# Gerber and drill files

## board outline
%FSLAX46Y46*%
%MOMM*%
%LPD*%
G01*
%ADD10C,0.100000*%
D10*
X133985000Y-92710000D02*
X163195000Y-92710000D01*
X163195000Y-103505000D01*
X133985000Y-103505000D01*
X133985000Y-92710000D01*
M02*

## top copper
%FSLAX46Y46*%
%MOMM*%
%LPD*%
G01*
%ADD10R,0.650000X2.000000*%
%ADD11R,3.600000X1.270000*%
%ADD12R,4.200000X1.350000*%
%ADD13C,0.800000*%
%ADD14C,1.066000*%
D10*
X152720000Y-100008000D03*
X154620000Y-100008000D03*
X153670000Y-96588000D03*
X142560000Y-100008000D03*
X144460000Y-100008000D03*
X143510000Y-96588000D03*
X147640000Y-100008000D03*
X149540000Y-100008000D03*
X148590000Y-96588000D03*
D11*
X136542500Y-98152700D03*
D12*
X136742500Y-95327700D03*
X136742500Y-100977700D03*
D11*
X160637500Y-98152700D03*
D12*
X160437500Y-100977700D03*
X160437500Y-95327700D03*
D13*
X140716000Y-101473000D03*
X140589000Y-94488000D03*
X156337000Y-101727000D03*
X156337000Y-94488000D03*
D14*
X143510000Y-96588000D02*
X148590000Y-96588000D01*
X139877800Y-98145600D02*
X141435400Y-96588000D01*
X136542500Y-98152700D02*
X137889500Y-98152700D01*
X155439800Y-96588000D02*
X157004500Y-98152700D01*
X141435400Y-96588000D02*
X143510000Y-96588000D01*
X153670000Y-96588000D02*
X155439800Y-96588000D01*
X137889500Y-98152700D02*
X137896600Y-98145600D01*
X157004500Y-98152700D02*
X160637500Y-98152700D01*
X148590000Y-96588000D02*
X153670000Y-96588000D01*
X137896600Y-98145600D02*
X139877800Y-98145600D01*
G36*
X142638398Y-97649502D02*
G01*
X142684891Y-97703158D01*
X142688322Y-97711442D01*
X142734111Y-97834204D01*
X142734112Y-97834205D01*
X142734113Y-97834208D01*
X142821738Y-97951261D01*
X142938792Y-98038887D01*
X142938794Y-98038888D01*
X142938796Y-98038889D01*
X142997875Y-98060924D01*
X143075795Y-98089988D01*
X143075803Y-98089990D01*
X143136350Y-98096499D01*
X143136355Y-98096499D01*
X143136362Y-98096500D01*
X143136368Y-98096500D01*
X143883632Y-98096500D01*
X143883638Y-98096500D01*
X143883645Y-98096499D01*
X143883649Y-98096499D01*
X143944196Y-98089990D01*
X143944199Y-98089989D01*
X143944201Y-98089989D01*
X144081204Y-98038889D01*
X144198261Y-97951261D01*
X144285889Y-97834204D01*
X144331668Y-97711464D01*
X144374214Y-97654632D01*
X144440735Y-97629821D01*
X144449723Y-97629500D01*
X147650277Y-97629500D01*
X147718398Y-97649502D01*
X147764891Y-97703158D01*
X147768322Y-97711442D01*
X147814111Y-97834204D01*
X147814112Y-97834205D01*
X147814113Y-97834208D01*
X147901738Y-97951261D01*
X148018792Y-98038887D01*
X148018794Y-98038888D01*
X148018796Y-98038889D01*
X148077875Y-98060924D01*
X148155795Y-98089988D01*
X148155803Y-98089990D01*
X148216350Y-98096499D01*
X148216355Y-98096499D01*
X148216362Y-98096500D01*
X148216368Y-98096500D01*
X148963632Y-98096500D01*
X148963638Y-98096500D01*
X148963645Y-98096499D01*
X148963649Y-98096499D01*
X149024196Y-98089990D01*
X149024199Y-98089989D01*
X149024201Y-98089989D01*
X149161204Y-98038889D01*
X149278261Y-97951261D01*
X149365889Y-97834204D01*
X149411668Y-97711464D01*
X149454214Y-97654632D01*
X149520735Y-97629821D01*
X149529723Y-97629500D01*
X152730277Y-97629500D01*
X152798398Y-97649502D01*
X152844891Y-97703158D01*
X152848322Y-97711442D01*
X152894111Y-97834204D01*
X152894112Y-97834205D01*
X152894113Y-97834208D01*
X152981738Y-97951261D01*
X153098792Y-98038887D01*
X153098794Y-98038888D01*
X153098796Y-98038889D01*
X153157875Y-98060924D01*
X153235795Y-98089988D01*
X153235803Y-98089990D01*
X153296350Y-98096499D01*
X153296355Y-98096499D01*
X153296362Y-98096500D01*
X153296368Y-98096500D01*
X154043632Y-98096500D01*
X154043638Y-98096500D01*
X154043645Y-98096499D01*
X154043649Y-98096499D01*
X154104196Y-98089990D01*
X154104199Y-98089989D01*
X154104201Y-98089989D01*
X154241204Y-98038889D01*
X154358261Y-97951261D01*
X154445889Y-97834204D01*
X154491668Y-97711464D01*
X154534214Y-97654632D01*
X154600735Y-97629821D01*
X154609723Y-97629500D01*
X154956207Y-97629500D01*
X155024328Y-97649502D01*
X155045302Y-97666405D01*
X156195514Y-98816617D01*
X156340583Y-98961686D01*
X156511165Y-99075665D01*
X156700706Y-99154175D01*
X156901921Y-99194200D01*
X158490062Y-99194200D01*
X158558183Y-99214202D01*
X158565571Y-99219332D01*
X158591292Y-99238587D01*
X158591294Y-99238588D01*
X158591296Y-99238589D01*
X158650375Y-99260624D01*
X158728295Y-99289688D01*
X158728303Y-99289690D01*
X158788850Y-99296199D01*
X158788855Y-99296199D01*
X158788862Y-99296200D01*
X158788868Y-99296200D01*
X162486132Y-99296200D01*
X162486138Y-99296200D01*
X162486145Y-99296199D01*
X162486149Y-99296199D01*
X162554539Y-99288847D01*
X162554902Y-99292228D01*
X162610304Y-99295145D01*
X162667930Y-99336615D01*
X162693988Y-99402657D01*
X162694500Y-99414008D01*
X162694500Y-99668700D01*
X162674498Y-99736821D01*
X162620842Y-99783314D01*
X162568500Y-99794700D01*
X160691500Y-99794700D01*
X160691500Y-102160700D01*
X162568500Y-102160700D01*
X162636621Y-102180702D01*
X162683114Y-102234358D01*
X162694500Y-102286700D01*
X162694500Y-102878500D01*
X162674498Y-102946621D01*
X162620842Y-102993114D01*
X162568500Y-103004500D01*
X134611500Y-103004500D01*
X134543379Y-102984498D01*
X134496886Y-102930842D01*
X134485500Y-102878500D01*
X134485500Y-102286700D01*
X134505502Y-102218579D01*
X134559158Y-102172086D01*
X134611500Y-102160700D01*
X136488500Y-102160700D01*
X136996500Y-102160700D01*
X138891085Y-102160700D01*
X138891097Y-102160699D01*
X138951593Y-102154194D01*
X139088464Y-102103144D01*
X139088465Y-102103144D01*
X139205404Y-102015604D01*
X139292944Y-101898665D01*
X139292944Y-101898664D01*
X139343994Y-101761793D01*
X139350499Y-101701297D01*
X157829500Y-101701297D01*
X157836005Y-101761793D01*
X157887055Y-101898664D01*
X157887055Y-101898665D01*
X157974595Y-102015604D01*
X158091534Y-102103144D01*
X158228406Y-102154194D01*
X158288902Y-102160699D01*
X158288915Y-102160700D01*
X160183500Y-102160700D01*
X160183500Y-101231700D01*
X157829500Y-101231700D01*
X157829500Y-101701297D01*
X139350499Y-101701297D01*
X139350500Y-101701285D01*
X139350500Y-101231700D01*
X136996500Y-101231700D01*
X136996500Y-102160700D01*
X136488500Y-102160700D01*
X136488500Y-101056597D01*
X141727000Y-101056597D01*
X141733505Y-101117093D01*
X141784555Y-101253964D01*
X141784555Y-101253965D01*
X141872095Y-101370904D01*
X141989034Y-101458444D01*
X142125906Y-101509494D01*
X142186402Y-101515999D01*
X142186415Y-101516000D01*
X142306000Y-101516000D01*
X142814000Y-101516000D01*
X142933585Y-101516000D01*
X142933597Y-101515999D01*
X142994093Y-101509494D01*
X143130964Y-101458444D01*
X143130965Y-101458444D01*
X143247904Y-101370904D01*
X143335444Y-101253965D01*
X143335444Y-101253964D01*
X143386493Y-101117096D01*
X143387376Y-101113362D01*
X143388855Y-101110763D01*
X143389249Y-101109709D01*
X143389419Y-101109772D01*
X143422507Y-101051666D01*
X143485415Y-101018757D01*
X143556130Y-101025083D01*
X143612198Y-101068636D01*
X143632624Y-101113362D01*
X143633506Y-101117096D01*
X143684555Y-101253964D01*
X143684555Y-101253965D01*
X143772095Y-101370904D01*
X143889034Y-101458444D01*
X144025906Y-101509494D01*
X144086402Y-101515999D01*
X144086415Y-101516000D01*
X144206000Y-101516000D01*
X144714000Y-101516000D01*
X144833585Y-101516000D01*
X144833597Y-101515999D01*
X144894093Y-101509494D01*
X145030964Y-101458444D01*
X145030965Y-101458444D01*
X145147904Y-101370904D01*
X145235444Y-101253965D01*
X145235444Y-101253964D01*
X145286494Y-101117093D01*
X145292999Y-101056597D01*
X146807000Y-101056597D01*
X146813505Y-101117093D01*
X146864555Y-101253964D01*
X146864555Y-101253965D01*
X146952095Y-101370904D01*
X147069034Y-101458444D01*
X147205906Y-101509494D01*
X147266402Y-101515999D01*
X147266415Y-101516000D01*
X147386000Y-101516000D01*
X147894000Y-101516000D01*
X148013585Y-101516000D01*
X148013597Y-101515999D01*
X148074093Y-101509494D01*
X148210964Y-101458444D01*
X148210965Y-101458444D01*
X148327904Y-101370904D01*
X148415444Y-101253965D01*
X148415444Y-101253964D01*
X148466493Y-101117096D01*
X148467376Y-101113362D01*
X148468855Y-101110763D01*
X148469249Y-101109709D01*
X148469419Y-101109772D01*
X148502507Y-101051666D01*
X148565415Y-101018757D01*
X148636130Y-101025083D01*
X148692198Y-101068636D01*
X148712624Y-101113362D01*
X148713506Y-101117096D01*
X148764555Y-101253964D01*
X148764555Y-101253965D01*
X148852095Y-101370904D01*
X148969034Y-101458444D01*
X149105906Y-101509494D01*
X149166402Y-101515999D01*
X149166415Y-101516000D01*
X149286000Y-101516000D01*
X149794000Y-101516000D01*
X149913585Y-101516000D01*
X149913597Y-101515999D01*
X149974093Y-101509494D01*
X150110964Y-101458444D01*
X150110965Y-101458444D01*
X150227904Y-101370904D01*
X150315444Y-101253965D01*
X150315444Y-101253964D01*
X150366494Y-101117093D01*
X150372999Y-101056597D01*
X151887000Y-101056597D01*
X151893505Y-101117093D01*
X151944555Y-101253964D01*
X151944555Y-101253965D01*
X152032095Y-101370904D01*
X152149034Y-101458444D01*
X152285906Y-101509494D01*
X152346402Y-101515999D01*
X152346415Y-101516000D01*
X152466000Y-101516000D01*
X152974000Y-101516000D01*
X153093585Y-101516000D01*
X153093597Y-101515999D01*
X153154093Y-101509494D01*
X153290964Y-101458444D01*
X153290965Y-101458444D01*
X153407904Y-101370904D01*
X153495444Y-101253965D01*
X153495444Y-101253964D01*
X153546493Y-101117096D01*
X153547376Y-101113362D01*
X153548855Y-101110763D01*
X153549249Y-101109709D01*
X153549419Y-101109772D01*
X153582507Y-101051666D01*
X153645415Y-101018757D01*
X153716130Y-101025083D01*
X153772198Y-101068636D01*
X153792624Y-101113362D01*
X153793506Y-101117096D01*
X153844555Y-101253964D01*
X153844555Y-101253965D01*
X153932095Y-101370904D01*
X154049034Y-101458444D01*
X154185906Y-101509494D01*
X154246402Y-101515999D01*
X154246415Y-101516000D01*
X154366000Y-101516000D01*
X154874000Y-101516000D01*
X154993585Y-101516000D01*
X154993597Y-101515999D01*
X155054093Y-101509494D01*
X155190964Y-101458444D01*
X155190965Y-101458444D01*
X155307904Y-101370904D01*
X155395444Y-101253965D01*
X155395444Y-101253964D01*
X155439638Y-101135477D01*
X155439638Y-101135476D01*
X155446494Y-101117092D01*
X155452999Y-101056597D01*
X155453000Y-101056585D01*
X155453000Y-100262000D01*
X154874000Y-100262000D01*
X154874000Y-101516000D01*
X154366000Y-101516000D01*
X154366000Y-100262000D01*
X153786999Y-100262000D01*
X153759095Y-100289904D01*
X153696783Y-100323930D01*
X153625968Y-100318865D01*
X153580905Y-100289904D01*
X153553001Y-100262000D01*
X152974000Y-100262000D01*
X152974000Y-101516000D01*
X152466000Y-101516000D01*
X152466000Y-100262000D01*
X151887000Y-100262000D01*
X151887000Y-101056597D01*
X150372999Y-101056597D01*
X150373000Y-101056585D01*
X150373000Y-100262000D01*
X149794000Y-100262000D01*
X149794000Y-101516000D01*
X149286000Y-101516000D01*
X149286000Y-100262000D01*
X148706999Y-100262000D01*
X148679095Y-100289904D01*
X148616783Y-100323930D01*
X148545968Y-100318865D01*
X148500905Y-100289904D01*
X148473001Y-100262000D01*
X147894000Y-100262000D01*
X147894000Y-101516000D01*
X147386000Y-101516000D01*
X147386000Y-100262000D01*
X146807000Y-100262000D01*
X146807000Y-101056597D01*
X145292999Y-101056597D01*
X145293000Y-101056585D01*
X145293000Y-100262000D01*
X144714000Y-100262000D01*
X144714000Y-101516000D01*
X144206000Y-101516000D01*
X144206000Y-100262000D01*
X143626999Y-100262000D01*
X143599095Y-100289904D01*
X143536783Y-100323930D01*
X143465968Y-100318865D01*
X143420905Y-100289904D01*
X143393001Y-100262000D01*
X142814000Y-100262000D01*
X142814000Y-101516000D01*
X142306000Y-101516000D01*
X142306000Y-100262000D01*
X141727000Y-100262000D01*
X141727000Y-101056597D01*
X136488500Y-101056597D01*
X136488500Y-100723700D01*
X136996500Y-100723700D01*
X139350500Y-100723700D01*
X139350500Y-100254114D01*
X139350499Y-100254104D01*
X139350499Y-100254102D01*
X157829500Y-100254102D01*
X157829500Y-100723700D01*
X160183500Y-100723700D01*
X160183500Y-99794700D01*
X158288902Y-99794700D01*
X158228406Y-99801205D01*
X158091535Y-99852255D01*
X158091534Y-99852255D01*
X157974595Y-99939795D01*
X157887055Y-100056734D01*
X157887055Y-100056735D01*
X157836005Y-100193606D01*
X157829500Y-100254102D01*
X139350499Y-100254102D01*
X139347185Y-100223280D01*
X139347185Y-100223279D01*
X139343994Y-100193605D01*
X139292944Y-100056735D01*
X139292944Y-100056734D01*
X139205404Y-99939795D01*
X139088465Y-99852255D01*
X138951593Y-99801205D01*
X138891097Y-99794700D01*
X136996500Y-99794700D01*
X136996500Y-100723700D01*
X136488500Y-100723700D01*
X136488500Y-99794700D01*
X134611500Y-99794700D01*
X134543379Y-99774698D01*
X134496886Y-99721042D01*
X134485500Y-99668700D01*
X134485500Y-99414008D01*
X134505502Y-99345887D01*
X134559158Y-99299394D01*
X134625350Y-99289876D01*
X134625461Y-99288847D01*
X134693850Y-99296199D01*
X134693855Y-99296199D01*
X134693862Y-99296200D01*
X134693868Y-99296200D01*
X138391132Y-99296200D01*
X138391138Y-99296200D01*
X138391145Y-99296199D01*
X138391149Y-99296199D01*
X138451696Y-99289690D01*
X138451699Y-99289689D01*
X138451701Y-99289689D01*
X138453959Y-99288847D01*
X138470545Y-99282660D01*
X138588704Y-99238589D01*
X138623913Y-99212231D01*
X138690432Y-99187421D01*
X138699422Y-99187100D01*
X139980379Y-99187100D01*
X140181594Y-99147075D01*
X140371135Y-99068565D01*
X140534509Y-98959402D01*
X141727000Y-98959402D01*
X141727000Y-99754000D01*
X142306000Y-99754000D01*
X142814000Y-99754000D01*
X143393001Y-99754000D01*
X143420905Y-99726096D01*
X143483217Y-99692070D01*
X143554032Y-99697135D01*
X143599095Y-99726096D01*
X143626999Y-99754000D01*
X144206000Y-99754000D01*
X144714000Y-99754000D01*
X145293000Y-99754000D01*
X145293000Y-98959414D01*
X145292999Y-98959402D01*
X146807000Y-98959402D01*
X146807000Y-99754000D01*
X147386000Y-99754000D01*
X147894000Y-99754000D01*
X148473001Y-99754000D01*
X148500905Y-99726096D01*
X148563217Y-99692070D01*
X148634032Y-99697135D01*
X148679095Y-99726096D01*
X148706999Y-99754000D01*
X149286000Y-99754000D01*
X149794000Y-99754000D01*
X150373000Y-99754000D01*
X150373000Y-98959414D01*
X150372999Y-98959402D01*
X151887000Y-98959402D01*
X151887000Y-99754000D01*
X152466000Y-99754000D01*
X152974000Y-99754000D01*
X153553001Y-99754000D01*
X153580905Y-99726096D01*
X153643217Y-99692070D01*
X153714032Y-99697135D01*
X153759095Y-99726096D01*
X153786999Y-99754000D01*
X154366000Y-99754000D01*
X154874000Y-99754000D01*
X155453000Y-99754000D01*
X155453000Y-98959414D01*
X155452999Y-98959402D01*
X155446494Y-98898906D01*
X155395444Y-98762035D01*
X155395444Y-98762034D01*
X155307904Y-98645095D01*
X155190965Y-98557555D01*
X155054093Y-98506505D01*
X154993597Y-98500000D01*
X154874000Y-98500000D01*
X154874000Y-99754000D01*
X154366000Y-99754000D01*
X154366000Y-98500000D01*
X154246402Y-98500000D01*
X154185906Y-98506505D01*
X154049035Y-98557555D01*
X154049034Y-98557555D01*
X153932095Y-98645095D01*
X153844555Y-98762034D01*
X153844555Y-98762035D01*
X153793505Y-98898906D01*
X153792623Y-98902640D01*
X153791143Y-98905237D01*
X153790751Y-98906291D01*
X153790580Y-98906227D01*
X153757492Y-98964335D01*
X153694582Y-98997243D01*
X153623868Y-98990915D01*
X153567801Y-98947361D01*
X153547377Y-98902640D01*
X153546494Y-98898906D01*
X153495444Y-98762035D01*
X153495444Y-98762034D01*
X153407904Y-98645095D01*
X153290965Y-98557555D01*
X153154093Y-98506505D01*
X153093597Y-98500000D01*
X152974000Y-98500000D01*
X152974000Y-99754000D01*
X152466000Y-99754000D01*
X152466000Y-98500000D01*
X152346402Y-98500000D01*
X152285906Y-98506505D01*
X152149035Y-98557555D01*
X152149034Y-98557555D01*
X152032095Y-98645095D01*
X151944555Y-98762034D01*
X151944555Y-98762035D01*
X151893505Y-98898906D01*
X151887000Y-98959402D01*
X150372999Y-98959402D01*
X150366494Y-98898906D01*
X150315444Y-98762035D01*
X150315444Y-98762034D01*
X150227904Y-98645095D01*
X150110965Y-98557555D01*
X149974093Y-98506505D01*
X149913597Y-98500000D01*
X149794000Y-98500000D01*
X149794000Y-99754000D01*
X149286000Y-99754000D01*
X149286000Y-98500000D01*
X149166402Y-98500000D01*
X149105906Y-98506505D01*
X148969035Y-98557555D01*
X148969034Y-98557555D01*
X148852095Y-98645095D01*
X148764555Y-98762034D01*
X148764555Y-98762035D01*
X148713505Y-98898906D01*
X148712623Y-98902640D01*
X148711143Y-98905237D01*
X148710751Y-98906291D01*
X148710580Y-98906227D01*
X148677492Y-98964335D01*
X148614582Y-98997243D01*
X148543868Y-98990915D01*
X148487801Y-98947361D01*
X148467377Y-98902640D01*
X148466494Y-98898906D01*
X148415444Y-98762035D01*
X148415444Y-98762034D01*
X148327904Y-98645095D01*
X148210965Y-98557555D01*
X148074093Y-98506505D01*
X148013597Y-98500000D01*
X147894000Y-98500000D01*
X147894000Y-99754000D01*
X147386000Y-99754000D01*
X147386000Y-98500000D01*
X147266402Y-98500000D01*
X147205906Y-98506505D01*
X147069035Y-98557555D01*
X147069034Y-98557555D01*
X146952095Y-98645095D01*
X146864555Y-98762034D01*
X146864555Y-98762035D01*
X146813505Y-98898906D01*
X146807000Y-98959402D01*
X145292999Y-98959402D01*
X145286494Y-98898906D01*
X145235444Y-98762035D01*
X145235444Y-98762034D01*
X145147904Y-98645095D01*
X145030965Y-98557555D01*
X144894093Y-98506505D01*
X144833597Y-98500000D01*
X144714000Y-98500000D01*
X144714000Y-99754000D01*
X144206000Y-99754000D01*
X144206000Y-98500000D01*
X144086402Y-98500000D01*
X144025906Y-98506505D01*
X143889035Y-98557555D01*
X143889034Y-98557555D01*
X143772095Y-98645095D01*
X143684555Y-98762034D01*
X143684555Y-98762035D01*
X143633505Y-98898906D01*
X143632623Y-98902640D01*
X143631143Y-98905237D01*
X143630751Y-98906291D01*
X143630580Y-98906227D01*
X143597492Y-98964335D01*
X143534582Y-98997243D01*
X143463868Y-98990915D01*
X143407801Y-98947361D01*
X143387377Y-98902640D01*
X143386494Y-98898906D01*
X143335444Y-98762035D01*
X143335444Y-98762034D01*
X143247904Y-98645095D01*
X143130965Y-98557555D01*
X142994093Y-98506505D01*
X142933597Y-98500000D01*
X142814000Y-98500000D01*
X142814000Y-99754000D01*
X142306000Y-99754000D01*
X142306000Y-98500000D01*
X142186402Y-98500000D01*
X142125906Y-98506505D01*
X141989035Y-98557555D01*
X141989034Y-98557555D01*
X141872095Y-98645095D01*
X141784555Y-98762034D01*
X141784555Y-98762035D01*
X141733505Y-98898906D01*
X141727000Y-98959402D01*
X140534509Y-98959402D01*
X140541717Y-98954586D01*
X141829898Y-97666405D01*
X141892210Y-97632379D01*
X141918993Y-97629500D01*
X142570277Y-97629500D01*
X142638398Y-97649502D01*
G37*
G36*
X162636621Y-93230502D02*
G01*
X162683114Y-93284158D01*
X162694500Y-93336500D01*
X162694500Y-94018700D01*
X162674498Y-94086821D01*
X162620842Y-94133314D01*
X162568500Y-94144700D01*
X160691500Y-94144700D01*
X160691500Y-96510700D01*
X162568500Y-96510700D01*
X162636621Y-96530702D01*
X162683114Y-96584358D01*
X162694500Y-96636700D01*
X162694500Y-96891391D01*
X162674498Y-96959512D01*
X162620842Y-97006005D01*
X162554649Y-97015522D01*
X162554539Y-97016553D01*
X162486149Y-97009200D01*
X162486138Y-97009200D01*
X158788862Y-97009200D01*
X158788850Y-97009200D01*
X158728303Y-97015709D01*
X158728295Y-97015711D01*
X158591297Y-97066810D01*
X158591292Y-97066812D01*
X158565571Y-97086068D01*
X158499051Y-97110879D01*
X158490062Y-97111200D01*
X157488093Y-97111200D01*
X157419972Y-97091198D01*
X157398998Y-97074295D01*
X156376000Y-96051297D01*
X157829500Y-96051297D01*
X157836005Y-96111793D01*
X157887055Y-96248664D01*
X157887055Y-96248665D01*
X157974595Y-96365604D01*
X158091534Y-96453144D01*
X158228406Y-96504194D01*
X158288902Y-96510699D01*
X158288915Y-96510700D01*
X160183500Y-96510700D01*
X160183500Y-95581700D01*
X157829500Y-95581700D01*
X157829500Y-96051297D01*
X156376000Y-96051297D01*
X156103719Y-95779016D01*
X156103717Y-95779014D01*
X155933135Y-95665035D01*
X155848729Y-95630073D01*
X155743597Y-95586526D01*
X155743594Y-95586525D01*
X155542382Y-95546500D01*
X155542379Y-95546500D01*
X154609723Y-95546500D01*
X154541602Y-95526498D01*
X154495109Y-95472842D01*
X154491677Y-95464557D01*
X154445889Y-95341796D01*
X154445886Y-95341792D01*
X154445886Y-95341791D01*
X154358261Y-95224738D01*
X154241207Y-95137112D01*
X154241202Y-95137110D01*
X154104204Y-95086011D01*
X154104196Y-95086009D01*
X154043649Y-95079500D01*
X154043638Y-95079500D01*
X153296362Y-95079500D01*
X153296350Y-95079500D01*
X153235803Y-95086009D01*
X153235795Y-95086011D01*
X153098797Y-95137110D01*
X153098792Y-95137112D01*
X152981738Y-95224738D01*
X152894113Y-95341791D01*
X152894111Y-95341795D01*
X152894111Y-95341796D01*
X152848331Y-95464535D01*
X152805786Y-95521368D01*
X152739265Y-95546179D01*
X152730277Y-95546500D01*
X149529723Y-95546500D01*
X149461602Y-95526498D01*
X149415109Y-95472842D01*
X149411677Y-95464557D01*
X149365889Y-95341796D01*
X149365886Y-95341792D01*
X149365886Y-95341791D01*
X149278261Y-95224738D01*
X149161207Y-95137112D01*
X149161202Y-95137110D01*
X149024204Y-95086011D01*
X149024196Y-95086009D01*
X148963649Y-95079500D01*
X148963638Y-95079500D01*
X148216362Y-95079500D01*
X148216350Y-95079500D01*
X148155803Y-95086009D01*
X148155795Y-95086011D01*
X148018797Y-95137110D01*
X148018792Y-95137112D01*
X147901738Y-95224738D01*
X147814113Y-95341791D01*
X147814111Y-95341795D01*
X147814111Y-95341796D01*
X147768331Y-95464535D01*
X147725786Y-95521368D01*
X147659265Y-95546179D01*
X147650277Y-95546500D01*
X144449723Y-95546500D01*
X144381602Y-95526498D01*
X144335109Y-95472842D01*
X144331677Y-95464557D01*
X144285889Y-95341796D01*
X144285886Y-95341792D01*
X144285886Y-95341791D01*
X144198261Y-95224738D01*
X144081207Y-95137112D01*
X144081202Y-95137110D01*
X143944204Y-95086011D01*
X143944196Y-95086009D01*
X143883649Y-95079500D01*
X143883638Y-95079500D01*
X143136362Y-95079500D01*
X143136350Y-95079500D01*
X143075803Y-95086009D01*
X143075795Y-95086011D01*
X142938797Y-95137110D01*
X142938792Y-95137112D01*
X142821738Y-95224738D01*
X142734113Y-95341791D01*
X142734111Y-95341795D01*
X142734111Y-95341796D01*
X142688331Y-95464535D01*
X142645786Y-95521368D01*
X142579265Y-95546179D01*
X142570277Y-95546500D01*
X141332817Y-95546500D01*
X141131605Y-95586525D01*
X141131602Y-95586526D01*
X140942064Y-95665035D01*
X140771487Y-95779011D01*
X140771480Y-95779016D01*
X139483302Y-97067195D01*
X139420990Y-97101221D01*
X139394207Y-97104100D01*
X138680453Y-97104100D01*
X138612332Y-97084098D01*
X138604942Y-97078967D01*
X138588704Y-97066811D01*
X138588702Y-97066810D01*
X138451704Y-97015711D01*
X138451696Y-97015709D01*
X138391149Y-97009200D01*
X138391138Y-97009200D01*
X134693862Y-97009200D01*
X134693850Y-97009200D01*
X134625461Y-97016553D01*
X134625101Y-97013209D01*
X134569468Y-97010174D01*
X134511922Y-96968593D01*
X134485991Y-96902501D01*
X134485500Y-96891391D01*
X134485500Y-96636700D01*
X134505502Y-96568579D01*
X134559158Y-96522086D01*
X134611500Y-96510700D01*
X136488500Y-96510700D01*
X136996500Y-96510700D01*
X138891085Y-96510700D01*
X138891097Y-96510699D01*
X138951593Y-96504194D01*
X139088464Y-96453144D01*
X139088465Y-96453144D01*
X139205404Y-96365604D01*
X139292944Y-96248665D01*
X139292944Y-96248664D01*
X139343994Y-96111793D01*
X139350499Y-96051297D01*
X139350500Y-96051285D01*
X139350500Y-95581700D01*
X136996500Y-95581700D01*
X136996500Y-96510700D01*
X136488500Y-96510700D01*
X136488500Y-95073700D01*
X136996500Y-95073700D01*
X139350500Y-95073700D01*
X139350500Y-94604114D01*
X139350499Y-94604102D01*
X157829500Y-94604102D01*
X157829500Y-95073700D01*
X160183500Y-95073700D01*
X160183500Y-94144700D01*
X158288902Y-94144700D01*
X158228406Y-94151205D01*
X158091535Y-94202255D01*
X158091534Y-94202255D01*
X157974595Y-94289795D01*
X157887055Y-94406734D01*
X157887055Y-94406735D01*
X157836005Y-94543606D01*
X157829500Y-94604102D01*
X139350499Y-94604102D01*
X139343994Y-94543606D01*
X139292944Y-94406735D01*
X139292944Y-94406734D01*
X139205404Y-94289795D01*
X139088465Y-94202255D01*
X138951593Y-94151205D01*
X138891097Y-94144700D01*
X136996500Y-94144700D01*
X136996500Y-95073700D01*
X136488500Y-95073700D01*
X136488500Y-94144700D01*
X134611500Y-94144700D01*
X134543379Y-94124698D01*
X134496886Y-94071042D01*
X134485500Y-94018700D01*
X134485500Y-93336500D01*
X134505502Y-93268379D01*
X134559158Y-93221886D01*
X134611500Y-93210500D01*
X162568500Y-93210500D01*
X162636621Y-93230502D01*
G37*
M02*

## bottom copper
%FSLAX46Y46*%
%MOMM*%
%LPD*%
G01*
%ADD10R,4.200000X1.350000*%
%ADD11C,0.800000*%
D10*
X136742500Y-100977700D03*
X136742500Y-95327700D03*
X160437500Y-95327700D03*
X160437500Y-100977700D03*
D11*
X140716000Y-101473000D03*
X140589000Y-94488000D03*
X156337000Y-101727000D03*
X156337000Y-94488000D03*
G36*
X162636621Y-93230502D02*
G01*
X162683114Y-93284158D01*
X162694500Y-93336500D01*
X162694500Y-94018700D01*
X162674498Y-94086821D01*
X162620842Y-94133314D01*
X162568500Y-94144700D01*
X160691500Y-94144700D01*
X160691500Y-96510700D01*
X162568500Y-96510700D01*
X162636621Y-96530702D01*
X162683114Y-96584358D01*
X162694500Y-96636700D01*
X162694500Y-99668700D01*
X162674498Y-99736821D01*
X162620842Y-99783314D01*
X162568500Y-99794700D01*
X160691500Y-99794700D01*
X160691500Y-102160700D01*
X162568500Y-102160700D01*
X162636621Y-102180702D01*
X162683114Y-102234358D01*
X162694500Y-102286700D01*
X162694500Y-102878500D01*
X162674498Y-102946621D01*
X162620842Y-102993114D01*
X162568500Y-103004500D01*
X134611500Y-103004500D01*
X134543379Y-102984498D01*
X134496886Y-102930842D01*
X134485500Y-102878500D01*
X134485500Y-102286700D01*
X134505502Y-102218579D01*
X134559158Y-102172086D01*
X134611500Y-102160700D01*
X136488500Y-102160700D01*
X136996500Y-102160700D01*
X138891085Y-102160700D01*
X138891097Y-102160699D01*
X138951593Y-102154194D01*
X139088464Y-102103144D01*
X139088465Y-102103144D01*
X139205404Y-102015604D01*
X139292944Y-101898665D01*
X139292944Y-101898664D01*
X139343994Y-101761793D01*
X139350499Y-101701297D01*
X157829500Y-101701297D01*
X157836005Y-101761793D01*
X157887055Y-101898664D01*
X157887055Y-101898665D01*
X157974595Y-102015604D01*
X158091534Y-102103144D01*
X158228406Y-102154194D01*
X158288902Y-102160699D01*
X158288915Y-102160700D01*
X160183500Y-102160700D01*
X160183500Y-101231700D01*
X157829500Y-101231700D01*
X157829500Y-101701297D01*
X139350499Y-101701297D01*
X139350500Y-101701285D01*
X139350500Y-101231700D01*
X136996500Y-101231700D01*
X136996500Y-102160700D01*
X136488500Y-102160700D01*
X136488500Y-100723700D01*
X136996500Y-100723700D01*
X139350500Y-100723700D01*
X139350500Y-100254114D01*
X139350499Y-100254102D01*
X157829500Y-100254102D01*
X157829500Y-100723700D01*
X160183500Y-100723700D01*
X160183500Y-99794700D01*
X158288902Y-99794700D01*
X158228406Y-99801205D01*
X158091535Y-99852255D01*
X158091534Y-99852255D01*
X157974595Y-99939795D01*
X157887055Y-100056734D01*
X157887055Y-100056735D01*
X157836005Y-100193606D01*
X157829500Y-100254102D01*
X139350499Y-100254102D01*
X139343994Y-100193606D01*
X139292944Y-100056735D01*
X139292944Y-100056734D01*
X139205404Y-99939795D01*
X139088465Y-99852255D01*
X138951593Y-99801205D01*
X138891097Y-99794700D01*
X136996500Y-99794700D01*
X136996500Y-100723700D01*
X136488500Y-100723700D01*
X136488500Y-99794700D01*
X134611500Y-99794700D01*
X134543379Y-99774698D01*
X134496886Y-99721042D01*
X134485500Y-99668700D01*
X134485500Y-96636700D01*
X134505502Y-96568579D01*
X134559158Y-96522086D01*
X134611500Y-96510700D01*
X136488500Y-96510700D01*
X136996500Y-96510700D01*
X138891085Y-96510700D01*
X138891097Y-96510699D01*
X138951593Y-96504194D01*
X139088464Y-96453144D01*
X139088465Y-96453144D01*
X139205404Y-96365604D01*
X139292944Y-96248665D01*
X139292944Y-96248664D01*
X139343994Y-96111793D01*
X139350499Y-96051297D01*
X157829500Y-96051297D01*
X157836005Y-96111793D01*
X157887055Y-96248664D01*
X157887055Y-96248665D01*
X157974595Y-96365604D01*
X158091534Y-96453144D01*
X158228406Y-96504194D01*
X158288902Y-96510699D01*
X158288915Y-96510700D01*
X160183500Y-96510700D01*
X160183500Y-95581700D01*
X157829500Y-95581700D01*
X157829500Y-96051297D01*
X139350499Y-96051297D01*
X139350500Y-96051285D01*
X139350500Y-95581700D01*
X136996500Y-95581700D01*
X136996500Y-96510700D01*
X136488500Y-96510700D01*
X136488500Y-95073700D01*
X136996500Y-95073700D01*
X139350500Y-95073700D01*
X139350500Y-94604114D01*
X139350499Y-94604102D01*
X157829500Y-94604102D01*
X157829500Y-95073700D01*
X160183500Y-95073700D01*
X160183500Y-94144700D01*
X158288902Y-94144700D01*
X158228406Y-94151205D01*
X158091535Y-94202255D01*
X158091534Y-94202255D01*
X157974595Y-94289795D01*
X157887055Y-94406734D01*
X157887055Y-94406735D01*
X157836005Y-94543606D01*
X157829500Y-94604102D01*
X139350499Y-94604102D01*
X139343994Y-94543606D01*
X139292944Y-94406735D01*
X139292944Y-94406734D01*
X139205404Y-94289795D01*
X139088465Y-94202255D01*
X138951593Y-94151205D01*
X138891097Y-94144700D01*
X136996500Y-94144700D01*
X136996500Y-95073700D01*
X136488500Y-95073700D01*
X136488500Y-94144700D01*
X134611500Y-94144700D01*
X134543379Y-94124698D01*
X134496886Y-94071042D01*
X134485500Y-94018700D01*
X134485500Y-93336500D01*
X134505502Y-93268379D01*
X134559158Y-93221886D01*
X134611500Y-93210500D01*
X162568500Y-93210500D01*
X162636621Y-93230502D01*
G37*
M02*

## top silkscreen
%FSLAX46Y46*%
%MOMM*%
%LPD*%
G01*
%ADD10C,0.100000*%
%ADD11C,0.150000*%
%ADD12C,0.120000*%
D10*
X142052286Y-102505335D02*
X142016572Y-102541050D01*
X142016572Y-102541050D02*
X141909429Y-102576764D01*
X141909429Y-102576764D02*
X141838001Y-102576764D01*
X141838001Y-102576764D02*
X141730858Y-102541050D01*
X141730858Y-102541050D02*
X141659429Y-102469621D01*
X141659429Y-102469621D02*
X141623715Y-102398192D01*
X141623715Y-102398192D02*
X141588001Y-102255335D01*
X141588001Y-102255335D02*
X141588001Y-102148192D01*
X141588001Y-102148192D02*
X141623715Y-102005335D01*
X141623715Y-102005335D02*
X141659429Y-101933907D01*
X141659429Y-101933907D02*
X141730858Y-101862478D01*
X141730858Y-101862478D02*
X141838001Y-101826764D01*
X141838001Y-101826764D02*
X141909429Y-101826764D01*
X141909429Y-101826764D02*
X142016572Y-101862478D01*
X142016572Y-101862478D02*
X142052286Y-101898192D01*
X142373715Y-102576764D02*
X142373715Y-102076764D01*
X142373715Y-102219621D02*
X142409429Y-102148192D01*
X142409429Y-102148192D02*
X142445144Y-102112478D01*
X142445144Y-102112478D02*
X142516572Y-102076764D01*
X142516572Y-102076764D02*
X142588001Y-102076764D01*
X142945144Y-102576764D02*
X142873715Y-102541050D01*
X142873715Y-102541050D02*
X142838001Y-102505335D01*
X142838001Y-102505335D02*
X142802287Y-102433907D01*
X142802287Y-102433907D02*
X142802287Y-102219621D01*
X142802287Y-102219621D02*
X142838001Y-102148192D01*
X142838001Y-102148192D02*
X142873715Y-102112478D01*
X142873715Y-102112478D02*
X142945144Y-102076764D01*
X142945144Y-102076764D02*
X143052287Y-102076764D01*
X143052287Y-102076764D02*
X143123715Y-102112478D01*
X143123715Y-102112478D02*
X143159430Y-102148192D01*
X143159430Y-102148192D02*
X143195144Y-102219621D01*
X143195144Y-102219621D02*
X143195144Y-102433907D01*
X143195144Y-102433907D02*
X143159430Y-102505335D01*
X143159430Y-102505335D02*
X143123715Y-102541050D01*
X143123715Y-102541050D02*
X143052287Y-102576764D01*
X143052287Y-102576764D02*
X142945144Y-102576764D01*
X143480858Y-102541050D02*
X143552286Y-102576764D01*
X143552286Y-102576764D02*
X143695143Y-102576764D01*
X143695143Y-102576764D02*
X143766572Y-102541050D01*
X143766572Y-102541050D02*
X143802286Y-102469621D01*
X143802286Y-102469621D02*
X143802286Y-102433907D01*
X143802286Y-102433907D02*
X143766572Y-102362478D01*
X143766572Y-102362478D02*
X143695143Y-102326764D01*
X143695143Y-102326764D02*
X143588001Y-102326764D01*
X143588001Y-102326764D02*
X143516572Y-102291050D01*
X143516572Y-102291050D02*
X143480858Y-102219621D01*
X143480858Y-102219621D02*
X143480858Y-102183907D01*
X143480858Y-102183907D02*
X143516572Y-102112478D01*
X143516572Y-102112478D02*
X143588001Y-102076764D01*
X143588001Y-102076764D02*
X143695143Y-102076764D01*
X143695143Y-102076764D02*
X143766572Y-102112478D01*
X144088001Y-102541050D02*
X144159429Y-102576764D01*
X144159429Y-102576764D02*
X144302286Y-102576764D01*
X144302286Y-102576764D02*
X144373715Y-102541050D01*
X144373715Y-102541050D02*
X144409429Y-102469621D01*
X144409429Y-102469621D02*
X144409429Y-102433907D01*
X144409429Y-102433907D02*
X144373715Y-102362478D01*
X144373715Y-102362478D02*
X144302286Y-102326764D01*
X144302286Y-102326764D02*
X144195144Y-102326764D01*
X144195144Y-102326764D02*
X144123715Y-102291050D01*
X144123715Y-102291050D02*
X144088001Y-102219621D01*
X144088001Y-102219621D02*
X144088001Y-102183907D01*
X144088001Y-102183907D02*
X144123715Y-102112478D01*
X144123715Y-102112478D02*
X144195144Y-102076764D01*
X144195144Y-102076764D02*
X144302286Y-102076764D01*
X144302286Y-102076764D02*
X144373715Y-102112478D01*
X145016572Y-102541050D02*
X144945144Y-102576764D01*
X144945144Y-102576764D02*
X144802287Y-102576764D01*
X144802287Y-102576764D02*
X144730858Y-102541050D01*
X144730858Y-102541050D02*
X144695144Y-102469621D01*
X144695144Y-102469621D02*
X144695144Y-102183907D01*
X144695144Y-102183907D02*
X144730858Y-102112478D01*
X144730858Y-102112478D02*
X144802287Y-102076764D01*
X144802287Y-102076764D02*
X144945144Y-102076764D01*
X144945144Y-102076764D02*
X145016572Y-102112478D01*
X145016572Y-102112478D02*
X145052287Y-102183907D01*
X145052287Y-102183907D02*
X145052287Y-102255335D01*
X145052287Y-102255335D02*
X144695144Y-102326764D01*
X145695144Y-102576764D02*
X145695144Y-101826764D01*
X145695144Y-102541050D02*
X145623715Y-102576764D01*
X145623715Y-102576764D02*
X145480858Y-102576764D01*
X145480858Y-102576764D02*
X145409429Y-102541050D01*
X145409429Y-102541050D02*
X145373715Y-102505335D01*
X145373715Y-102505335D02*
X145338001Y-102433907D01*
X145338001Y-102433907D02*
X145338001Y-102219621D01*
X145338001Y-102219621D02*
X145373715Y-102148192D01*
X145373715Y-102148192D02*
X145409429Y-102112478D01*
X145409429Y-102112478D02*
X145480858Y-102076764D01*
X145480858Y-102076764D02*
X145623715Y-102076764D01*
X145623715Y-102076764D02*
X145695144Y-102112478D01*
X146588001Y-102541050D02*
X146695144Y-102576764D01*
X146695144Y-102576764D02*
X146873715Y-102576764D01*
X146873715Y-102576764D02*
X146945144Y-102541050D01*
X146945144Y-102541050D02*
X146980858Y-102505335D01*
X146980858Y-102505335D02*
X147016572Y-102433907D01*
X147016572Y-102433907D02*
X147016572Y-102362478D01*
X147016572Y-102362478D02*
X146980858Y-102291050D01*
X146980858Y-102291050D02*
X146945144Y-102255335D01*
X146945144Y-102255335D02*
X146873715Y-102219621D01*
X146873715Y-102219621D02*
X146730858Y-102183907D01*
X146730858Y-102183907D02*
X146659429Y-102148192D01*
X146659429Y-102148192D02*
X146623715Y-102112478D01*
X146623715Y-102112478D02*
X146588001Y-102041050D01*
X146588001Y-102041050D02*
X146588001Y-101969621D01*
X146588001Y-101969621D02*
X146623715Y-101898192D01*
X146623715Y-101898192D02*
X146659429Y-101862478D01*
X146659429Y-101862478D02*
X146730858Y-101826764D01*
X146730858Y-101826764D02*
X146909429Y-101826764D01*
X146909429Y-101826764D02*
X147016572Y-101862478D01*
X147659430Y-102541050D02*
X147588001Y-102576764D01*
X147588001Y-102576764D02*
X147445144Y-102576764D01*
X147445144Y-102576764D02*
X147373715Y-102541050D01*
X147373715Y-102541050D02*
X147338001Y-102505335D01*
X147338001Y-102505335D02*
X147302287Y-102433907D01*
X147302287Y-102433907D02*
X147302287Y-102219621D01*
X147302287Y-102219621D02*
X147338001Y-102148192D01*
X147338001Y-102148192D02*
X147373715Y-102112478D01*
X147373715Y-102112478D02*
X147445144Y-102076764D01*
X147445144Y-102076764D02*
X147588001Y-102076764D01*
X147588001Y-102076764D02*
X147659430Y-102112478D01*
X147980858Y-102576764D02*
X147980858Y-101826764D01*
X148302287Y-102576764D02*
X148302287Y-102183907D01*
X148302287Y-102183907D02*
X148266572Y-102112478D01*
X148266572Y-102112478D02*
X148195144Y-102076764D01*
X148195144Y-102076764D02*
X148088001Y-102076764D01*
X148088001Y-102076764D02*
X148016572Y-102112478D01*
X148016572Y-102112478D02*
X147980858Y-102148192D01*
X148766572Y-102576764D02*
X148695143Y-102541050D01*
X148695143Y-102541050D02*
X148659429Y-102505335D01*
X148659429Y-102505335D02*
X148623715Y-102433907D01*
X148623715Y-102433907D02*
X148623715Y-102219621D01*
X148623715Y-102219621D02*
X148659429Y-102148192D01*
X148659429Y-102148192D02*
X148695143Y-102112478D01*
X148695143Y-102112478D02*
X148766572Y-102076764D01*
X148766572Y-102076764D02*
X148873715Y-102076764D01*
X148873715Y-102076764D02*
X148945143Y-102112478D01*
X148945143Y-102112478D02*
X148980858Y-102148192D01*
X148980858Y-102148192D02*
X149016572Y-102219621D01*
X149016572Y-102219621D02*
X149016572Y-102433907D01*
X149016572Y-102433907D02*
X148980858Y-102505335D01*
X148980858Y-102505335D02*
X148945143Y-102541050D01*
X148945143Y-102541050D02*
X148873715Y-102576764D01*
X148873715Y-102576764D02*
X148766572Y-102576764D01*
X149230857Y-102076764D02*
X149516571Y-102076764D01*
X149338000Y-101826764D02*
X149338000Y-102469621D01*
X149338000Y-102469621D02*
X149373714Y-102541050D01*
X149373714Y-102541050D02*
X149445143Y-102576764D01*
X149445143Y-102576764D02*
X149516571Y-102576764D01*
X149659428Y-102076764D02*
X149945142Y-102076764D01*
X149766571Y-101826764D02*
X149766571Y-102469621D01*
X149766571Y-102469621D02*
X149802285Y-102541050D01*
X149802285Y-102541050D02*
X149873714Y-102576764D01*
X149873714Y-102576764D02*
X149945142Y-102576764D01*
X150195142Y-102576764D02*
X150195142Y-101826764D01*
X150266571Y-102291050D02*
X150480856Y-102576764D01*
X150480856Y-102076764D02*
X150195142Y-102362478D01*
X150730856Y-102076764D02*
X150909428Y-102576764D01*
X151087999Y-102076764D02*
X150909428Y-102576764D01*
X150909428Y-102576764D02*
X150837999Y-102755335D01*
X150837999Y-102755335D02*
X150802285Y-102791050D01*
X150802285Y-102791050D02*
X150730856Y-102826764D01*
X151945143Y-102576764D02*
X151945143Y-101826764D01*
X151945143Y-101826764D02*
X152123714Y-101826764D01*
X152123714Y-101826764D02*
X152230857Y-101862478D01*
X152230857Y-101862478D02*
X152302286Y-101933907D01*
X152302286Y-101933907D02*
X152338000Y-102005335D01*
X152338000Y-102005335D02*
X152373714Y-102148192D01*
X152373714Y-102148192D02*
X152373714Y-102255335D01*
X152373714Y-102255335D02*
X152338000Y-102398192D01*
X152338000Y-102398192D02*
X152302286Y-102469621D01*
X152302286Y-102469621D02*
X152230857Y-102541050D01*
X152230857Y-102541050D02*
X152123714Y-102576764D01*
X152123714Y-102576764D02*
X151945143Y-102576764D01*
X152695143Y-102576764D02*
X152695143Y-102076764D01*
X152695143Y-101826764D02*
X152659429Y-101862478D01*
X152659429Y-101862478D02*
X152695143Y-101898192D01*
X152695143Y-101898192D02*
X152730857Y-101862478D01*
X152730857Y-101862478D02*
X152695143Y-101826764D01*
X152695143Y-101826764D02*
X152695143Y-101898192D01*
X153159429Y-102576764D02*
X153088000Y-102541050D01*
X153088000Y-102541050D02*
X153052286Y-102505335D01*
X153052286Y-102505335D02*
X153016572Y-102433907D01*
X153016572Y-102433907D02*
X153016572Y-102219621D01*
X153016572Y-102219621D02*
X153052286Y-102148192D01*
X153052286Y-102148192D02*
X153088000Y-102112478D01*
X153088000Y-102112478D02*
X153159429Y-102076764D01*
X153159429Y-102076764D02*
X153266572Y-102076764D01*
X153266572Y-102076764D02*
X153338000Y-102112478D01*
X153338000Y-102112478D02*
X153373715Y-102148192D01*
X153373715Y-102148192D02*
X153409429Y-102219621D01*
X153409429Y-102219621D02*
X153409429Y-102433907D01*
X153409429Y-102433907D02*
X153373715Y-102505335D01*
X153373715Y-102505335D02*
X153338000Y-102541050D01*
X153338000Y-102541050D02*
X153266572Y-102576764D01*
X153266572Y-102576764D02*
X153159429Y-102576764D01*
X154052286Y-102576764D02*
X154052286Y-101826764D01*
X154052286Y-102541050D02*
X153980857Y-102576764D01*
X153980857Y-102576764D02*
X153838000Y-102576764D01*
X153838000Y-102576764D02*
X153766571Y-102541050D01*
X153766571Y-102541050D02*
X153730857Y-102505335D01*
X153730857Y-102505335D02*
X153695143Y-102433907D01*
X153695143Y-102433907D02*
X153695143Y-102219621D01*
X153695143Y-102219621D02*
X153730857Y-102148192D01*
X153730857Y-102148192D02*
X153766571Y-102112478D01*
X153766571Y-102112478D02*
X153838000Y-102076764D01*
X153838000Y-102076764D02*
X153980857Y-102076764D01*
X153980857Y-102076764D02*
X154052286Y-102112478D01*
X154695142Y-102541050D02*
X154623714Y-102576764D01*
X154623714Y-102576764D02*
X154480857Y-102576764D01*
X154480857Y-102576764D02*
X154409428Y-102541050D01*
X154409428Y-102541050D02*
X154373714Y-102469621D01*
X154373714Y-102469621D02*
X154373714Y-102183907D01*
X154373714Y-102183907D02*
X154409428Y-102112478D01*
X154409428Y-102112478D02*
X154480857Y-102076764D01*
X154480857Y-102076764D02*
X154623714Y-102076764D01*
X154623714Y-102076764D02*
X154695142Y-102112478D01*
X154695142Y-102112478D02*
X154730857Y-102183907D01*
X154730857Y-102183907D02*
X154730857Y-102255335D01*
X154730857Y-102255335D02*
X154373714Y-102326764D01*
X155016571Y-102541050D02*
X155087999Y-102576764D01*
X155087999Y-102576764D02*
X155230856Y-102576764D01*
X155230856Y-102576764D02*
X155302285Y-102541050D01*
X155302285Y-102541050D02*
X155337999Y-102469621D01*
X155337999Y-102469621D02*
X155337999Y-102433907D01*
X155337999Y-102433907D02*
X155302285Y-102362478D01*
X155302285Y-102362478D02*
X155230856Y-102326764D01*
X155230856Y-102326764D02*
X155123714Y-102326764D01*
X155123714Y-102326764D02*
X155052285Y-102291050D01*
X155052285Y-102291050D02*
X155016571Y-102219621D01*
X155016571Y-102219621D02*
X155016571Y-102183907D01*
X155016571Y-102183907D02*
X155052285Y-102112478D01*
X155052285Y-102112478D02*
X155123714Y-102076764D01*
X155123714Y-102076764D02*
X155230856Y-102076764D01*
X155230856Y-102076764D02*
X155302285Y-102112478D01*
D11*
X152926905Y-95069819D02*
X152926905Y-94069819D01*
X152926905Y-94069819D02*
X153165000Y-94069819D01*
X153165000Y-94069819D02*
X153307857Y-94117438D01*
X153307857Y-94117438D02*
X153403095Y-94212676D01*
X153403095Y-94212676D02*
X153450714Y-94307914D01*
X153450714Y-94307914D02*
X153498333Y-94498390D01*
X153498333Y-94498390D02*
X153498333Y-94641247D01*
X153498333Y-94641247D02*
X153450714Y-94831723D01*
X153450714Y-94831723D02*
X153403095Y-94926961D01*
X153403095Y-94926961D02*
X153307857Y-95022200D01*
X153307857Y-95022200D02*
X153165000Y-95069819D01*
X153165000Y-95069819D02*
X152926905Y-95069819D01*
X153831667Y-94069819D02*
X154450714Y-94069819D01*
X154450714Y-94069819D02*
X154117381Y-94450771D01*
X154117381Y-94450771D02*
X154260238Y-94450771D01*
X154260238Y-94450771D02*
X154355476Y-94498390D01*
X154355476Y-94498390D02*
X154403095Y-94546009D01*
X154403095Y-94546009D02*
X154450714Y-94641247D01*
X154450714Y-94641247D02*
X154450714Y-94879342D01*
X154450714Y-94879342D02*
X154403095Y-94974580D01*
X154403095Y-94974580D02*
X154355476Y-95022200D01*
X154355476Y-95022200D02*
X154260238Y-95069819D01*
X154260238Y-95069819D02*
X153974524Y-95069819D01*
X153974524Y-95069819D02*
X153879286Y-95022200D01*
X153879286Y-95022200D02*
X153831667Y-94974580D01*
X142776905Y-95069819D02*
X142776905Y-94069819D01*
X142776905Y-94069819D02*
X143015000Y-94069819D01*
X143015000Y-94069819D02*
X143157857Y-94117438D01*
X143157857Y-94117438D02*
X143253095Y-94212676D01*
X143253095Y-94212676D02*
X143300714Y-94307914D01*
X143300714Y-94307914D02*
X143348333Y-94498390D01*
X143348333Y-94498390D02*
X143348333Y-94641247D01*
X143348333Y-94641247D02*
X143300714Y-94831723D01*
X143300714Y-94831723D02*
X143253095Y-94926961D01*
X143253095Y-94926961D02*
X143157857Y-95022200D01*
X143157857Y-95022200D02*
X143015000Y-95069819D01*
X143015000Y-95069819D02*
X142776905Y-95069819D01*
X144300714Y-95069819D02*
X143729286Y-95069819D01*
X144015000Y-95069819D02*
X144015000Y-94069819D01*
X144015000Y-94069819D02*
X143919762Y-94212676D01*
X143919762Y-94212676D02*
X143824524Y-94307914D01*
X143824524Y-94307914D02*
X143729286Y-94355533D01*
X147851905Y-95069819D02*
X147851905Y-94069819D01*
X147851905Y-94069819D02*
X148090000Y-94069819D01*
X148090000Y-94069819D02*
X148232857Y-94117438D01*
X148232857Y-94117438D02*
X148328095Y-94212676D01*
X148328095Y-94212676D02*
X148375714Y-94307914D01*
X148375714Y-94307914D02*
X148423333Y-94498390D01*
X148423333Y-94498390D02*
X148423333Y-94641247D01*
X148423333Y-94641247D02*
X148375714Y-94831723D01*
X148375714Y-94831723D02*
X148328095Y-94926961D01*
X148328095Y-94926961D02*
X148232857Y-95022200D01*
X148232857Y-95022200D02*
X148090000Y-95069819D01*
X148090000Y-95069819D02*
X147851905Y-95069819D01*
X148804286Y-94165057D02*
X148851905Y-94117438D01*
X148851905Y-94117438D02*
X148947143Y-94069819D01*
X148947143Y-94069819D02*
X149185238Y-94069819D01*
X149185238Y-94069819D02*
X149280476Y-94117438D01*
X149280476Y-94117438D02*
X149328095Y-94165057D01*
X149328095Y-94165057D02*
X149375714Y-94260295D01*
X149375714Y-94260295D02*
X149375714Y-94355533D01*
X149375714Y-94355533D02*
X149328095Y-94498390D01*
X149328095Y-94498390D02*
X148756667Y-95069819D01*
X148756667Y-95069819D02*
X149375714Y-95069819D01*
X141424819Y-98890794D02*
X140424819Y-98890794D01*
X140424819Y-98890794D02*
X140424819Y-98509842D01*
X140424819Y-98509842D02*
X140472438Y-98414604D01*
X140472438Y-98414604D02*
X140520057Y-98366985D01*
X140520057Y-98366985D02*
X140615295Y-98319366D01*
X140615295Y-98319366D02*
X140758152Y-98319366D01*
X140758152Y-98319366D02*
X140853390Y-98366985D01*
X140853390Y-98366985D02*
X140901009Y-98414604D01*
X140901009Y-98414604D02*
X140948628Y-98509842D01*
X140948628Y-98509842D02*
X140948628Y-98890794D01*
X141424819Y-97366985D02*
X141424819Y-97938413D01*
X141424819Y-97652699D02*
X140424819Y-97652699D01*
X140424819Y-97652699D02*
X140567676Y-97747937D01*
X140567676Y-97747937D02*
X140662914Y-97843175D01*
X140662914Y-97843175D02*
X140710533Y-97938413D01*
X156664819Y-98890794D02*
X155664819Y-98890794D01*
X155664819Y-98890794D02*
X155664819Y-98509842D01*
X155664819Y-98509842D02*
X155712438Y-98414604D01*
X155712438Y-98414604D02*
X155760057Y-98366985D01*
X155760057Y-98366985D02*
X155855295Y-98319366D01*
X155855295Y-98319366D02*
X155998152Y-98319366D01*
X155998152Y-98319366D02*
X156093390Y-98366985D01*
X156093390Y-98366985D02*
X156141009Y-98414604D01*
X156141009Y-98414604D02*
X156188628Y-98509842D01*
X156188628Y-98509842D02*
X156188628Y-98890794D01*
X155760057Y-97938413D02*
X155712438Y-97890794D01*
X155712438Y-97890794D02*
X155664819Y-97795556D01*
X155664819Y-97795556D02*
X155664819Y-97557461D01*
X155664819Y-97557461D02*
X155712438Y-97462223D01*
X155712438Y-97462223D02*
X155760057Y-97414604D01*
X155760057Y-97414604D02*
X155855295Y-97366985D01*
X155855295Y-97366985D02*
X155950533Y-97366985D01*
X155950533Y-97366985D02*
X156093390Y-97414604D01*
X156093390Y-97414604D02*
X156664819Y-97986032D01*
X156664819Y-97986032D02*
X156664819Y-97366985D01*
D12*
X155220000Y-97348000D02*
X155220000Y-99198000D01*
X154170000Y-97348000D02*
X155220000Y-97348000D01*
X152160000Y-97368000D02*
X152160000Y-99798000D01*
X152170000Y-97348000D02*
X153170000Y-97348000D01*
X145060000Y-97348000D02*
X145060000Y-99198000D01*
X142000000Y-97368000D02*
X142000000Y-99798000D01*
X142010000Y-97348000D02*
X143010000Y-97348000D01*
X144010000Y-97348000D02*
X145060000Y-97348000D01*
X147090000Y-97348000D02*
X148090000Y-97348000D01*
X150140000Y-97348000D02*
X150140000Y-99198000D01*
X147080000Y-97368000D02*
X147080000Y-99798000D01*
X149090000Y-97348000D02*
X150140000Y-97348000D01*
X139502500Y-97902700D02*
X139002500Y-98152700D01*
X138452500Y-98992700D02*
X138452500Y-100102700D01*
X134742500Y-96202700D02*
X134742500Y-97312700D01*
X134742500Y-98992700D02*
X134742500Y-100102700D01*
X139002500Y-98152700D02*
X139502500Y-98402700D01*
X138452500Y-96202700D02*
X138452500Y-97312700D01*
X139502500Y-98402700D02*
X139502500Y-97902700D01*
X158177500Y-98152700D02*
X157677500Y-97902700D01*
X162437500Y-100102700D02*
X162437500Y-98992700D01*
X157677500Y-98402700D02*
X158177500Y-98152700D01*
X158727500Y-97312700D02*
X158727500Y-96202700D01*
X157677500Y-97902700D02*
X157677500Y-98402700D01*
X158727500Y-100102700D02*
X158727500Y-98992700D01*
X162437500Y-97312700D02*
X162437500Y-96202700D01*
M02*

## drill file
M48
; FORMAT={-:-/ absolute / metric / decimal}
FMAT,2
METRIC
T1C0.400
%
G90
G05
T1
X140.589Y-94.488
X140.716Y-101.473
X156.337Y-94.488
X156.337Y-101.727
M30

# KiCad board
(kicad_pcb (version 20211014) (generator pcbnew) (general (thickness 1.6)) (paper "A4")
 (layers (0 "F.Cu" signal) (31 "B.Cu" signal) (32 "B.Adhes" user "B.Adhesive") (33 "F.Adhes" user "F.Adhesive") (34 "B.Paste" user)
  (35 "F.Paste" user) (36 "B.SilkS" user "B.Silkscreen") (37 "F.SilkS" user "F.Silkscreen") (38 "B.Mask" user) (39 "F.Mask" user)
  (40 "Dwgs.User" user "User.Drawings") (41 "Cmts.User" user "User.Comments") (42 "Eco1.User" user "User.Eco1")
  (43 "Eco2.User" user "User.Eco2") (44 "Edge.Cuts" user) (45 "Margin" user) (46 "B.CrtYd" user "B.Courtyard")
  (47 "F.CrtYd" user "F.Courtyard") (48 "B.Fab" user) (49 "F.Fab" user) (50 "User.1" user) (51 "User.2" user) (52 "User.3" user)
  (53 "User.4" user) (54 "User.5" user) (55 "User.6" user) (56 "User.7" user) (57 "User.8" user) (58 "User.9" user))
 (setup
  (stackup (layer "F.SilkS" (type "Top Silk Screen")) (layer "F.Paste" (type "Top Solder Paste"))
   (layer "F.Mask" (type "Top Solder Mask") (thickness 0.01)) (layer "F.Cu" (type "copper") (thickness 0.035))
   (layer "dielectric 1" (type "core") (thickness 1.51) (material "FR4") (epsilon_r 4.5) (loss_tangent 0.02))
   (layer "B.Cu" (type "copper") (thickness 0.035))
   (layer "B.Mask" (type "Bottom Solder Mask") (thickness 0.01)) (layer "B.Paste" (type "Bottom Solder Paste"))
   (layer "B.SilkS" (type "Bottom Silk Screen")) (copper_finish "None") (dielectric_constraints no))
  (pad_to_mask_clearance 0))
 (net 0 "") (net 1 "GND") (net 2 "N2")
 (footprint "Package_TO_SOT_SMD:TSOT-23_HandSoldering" (layer "F.Cu") (at 153.67 98.298 90)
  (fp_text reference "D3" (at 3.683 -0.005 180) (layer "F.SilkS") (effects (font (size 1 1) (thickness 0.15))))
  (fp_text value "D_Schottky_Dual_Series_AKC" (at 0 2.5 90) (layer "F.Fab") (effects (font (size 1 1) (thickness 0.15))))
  (fp_line (start 0.95 1.55) (end -0.9 1.55) (layer "F.SilkS") (width 0.12))
  (fp_line (start 0.95 0.5) (end 0.95 1.55) (layer "F.SilkS") (width 0.12))
  (fp_line (start 0.93 -1.51) (end -1.5 -1.51) (layer "F.SilkS") (width 0.12))
  (fp_line (start 0.95 -1.5) (end 0.95 -0.5) (layer "F.SilkS") (width 0.12))
  (pad "1" smd rect (at -1.71 -0.95 90) (size 2 0.65) (layers "F.Cu" "F.Paste" "F.Mask") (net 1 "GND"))
  (pad "2" smd rect (at -1.71 0.95 90) (size 2 0.65) (layers "F.Cu" "F.Paste" "F.Mask") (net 1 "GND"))
  (pad "D3" smd rect (at 1.71 0 90) (size 2 0.65) (layers "F.Cu" "F.Paste" "F.Mask") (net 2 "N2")))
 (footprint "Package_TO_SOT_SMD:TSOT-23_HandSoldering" (layer "F.Cu") (at 143.51 98.298 90)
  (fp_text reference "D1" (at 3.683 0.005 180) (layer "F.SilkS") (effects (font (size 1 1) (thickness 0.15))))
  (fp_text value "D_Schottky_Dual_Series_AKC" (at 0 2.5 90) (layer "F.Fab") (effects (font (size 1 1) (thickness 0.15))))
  (fp_line (start 0.95 1.55) (end -0.9 1.55) (layer "F.SilkS") (width 0.12))
  (fp_line (start 0.93 -1.51) (end -1.5 -1.51) (layer "F.SilkS") (width 0.12))
  (fp_line (start 0.95 -1.5) (end 0.95 -0.5) (layer "F.SilkS") (width 0.12))
  (fp_line (start 0.95 0.5) (end 0.95 1.55) (layer "F.SilkS") (width 0.12))
  (pad "1" smd rect (at -1.71 -0.95 90) (size 2 0.65) (layers "F.Cu" "F.Paste" "F.Mask") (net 1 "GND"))
  (pad "2" smd rect (at -1.71 0.95 90) (size 2 0.65) (layers "F.Cu" "F.Paste" "F.Mask") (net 1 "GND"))
  (pad "3" smd rect (at 1.71 0 90) (size 2 0.65) (layers "F.Cu" "F.Paste" "F.Mask") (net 2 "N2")))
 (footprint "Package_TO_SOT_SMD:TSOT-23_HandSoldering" (layer "F.Cu") (at 148.59 98.298 90)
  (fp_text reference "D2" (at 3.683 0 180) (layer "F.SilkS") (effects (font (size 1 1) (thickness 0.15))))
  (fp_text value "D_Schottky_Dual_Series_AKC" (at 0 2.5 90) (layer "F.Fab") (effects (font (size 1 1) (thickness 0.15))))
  (fp_line (start 0.95 -1.5) (end 0.95 -0.5) (layer "F.SilkS") (width 0.12))
  (fp_line (start 0.95 1.55) (end -0.9 1.55) (layer "F.SilkS") (width 0.12))
  (fp_line (start 0.93 -1.51) (end -1.5 -1.51) (layer "F.SilkS") (width 0.12))
  (fp_line (start 0.95 0.5) (end 0.95 1.55) (layer "F.SilkS") (width 0.12))
  (pad "1" smd rect (at -1.71 -0.95 90) (size 2 0.65) (layers "F.Cu" "F.Paste" "F.Mask") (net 1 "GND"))
  (pad "2" smd rect (at -1.71 0.95 90) (size 2 0.65) (layers "F.Cu" "F.Paste" "F.Mask") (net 1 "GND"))
  (pad "3" smd rect (at 1.71 0 90) (size 2 0.65) (layers "F.Cu" "F.Paste" "F.Mask") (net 2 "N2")))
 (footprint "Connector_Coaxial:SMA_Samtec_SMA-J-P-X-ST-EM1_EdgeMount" (layer "F.Cu") (at 136.7425 98.1527 -90)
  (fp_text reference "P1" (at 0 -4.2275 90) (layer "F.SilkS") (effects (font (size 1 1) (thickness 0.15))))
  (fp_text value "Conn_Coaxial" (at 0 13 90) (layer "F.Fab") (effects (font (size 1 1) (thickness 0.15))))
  (fp_line (start -0.25 -2.76) (end 0 -2.26) (layer "F.SilkS") (width 0.12))
  (fp_line (start 0.84 -1.71) (end 1.95 -1.71) (layer "F.SilkS") (width 0.12))
  (fp_line (start -1.95 2) (end -0.84 2) (layer "F.SilkS") (width 0.12))
  (fp_line (start 0.84 2) (end 1.95 2) (layer "F.SilkS") (width 0.12))
  (fp_line (start 0 -2.26) (end 0.25 -2.76) (layer "F.SilkS") (width 0.12))
  (fp_line (start -1.95 -1.71) (end -0.84 -1.71) (layer "F.SilkS") (width 0.12))
  (fp_line (start 0.25 -2.76) (end -0.25 -2.76) (layer "F.SilkS") (width 0.12))
  (pad "1" smd rect (at 0 0.2 270) (size 1.27 3.6) (layers "F.Cu" "F.Paste" "F.Mask") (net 2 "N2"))
  (pad "2" smd rect (at 2.825 0 270) (size 1.35 4.2) (layers "B.Cu" "B.Paste" "B.Mask") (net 1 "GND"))
  (pad "2" smd rect (at -2.825 0 270) (size 1.35 4.2) (layers "B.Cu" "B.Paste" "B.Mask") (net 1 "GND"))
  (pad "2" smd rect (at -2.825 0 270) (size 1.35 4.2) (layers "F.Cu" "F.Paste" "F.Mask") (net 1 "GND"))
  (pad "2" smd rect (at 2.825 0 270) (size 1.35 4.2) (layers "F.Cu" "F.Paste" "F.Mask") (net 1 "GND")))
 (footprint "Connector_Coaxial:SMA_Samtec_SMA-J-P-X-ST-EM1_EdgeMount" (layer "F.Cu") (at 160.4375 98.1527 90)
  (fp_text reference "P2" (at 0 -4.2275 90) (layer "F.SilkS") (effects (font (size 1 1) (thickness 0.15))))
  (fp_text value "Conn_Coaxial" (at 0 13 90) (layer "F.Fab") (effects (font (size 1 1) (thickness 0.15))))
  (fp_line (start 0 -2.26) (end 0.25 -2.76) (layer "F.SilkS") (width 0.12))
  (fp_line (start -1.95 2) (end -0.84 2) (layer "F.SilkS") (width 0.12))
  (fp_line (start -0.25 -2.76) (end 0 -2.26) (layer "F.SilkS") (width 0.12))
  (fp_line (start 0.84 -1.71) (end 1.95 -1.71) (layer "F.SilkS") (width 0.12))
  (fp_line (start 0.25 -2.76) (end -0.25 -2.76) (layer "F.SilkS") (width 0.12))
  (fp_line (start -1.95 -1.71) (end -0.84 -1.71) (layer "F.SilkS") (width 0.12))
  (fp_line (start 0.84 2) (end 1.95 2) (layer "F.SilkS") (width 0.12))
  (pad "1" smd rect (at 0 0.2 90) (size 1.27 3.6) (layers "F.Cu" "F.Paste" "F.Mask") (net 2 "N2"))
  (pad "2" smd rect (at -2.825 0 90) (size 1.35 4.2) (layers "F.Cu" "F.Paste" "F.Mask") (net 1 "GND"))
  (pad "2" smd rect (at 2.825 0 90) (size 1.35 4.2) (layers "F.Cu" "F.Paste" "F.Mask") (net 1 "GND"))
  (pad "2" smd rect (at 2.825 0 90) (size 1.35 4.2) (layers "B.Cu" "B.Paste" "B.Mask") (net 1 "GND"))
  (pad "2" smd rect (at -2.825 0 90) (size 1.35 4.2) (layers "B.Cu" "B.Paste" "B.Mask") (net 1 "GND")))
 (gr_rect (start 133.985 92.71) (end 163.195 103.505) (layer "Edge.Cuts") (width 0.1) (fill none))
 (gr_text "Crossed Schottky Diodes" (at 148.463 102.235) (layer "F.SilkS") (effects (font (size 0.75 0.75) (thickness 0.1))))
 (via (at 140.716 101.473) (size 0.8) (drill 0.4) (layers "F.Cu" "B.Cu") (free) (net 1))
 (via (at 140.589 94.488) (size 0.8) (drill 0.4) (layers "F.Cu" "B.Cu") (free) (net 1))
 (via (at 156.337 101.727) (size 0.8) (drill 0.4) (layers "F.Cu" "B.Cu") (free) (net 1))
 (via (at 156.337 94.488) (size 0.8) (drill 0.4) (layers "F.Cu" "B.Cu") (free) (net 1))
 (segment (start 143.51 96.588) (end 148.59 96.588) (width 1.066) (layer "F.Cu") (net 2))
 (segment (start 139.8778 98.1456) (end 141.4354 96.588) (width 1.066) (layer "F.Cu") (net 2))
 (segment (start 136.5425 98.1527) (end 137.8895 98.1527) (width 1.066) (layer "F.Cu") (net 2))
 (segment (start 155.4398 96.588) (end 157.0045 98.1527) (width 1.066) (layer "F.Cu") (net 2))
 (segment (start 141.4354 96.588) (end 143.51 96.588) (width 1.066) (layer "F.Cu") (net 2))
 (segment (start 153.67 96.588) (end 155.4398 96.588) (width 1.066) (layer "F.Cu") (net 2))
 (segment (start 137.8895 98.1527) (end 137.8966 98.1456) (width 1.066) (layer "F.Cu") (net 2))
 (segment (start 157.0045 98.1527) (end 160.6375 98.1527) (width 1.066) (layer "F.Cu") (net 2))
 (segment (start 148.59 96.588) (end 153.67 96.588) (width 1.066) (layer "F.Cu") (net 2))
 (segment (start 137.8966 98.1456) (end 139.8778 98.1456) (width 1.066) (layer "F.Cu") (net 2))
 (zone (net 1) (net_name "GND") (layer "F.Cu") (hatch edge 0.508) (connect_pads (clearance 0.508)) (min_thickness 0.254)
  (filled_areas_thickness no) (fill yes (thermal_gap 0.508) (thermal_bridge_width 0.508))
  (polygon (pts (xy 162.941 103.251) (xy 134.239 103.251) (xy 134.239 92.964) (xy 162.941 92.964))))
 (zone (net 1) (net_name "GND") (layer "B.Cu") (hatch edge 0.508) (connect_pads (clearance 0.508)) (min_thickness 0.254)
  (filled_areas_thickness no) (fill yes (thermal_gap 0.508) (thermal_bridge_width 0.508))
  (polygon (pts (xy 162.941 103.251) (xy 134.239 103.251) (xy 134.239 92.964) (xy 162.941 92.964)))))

